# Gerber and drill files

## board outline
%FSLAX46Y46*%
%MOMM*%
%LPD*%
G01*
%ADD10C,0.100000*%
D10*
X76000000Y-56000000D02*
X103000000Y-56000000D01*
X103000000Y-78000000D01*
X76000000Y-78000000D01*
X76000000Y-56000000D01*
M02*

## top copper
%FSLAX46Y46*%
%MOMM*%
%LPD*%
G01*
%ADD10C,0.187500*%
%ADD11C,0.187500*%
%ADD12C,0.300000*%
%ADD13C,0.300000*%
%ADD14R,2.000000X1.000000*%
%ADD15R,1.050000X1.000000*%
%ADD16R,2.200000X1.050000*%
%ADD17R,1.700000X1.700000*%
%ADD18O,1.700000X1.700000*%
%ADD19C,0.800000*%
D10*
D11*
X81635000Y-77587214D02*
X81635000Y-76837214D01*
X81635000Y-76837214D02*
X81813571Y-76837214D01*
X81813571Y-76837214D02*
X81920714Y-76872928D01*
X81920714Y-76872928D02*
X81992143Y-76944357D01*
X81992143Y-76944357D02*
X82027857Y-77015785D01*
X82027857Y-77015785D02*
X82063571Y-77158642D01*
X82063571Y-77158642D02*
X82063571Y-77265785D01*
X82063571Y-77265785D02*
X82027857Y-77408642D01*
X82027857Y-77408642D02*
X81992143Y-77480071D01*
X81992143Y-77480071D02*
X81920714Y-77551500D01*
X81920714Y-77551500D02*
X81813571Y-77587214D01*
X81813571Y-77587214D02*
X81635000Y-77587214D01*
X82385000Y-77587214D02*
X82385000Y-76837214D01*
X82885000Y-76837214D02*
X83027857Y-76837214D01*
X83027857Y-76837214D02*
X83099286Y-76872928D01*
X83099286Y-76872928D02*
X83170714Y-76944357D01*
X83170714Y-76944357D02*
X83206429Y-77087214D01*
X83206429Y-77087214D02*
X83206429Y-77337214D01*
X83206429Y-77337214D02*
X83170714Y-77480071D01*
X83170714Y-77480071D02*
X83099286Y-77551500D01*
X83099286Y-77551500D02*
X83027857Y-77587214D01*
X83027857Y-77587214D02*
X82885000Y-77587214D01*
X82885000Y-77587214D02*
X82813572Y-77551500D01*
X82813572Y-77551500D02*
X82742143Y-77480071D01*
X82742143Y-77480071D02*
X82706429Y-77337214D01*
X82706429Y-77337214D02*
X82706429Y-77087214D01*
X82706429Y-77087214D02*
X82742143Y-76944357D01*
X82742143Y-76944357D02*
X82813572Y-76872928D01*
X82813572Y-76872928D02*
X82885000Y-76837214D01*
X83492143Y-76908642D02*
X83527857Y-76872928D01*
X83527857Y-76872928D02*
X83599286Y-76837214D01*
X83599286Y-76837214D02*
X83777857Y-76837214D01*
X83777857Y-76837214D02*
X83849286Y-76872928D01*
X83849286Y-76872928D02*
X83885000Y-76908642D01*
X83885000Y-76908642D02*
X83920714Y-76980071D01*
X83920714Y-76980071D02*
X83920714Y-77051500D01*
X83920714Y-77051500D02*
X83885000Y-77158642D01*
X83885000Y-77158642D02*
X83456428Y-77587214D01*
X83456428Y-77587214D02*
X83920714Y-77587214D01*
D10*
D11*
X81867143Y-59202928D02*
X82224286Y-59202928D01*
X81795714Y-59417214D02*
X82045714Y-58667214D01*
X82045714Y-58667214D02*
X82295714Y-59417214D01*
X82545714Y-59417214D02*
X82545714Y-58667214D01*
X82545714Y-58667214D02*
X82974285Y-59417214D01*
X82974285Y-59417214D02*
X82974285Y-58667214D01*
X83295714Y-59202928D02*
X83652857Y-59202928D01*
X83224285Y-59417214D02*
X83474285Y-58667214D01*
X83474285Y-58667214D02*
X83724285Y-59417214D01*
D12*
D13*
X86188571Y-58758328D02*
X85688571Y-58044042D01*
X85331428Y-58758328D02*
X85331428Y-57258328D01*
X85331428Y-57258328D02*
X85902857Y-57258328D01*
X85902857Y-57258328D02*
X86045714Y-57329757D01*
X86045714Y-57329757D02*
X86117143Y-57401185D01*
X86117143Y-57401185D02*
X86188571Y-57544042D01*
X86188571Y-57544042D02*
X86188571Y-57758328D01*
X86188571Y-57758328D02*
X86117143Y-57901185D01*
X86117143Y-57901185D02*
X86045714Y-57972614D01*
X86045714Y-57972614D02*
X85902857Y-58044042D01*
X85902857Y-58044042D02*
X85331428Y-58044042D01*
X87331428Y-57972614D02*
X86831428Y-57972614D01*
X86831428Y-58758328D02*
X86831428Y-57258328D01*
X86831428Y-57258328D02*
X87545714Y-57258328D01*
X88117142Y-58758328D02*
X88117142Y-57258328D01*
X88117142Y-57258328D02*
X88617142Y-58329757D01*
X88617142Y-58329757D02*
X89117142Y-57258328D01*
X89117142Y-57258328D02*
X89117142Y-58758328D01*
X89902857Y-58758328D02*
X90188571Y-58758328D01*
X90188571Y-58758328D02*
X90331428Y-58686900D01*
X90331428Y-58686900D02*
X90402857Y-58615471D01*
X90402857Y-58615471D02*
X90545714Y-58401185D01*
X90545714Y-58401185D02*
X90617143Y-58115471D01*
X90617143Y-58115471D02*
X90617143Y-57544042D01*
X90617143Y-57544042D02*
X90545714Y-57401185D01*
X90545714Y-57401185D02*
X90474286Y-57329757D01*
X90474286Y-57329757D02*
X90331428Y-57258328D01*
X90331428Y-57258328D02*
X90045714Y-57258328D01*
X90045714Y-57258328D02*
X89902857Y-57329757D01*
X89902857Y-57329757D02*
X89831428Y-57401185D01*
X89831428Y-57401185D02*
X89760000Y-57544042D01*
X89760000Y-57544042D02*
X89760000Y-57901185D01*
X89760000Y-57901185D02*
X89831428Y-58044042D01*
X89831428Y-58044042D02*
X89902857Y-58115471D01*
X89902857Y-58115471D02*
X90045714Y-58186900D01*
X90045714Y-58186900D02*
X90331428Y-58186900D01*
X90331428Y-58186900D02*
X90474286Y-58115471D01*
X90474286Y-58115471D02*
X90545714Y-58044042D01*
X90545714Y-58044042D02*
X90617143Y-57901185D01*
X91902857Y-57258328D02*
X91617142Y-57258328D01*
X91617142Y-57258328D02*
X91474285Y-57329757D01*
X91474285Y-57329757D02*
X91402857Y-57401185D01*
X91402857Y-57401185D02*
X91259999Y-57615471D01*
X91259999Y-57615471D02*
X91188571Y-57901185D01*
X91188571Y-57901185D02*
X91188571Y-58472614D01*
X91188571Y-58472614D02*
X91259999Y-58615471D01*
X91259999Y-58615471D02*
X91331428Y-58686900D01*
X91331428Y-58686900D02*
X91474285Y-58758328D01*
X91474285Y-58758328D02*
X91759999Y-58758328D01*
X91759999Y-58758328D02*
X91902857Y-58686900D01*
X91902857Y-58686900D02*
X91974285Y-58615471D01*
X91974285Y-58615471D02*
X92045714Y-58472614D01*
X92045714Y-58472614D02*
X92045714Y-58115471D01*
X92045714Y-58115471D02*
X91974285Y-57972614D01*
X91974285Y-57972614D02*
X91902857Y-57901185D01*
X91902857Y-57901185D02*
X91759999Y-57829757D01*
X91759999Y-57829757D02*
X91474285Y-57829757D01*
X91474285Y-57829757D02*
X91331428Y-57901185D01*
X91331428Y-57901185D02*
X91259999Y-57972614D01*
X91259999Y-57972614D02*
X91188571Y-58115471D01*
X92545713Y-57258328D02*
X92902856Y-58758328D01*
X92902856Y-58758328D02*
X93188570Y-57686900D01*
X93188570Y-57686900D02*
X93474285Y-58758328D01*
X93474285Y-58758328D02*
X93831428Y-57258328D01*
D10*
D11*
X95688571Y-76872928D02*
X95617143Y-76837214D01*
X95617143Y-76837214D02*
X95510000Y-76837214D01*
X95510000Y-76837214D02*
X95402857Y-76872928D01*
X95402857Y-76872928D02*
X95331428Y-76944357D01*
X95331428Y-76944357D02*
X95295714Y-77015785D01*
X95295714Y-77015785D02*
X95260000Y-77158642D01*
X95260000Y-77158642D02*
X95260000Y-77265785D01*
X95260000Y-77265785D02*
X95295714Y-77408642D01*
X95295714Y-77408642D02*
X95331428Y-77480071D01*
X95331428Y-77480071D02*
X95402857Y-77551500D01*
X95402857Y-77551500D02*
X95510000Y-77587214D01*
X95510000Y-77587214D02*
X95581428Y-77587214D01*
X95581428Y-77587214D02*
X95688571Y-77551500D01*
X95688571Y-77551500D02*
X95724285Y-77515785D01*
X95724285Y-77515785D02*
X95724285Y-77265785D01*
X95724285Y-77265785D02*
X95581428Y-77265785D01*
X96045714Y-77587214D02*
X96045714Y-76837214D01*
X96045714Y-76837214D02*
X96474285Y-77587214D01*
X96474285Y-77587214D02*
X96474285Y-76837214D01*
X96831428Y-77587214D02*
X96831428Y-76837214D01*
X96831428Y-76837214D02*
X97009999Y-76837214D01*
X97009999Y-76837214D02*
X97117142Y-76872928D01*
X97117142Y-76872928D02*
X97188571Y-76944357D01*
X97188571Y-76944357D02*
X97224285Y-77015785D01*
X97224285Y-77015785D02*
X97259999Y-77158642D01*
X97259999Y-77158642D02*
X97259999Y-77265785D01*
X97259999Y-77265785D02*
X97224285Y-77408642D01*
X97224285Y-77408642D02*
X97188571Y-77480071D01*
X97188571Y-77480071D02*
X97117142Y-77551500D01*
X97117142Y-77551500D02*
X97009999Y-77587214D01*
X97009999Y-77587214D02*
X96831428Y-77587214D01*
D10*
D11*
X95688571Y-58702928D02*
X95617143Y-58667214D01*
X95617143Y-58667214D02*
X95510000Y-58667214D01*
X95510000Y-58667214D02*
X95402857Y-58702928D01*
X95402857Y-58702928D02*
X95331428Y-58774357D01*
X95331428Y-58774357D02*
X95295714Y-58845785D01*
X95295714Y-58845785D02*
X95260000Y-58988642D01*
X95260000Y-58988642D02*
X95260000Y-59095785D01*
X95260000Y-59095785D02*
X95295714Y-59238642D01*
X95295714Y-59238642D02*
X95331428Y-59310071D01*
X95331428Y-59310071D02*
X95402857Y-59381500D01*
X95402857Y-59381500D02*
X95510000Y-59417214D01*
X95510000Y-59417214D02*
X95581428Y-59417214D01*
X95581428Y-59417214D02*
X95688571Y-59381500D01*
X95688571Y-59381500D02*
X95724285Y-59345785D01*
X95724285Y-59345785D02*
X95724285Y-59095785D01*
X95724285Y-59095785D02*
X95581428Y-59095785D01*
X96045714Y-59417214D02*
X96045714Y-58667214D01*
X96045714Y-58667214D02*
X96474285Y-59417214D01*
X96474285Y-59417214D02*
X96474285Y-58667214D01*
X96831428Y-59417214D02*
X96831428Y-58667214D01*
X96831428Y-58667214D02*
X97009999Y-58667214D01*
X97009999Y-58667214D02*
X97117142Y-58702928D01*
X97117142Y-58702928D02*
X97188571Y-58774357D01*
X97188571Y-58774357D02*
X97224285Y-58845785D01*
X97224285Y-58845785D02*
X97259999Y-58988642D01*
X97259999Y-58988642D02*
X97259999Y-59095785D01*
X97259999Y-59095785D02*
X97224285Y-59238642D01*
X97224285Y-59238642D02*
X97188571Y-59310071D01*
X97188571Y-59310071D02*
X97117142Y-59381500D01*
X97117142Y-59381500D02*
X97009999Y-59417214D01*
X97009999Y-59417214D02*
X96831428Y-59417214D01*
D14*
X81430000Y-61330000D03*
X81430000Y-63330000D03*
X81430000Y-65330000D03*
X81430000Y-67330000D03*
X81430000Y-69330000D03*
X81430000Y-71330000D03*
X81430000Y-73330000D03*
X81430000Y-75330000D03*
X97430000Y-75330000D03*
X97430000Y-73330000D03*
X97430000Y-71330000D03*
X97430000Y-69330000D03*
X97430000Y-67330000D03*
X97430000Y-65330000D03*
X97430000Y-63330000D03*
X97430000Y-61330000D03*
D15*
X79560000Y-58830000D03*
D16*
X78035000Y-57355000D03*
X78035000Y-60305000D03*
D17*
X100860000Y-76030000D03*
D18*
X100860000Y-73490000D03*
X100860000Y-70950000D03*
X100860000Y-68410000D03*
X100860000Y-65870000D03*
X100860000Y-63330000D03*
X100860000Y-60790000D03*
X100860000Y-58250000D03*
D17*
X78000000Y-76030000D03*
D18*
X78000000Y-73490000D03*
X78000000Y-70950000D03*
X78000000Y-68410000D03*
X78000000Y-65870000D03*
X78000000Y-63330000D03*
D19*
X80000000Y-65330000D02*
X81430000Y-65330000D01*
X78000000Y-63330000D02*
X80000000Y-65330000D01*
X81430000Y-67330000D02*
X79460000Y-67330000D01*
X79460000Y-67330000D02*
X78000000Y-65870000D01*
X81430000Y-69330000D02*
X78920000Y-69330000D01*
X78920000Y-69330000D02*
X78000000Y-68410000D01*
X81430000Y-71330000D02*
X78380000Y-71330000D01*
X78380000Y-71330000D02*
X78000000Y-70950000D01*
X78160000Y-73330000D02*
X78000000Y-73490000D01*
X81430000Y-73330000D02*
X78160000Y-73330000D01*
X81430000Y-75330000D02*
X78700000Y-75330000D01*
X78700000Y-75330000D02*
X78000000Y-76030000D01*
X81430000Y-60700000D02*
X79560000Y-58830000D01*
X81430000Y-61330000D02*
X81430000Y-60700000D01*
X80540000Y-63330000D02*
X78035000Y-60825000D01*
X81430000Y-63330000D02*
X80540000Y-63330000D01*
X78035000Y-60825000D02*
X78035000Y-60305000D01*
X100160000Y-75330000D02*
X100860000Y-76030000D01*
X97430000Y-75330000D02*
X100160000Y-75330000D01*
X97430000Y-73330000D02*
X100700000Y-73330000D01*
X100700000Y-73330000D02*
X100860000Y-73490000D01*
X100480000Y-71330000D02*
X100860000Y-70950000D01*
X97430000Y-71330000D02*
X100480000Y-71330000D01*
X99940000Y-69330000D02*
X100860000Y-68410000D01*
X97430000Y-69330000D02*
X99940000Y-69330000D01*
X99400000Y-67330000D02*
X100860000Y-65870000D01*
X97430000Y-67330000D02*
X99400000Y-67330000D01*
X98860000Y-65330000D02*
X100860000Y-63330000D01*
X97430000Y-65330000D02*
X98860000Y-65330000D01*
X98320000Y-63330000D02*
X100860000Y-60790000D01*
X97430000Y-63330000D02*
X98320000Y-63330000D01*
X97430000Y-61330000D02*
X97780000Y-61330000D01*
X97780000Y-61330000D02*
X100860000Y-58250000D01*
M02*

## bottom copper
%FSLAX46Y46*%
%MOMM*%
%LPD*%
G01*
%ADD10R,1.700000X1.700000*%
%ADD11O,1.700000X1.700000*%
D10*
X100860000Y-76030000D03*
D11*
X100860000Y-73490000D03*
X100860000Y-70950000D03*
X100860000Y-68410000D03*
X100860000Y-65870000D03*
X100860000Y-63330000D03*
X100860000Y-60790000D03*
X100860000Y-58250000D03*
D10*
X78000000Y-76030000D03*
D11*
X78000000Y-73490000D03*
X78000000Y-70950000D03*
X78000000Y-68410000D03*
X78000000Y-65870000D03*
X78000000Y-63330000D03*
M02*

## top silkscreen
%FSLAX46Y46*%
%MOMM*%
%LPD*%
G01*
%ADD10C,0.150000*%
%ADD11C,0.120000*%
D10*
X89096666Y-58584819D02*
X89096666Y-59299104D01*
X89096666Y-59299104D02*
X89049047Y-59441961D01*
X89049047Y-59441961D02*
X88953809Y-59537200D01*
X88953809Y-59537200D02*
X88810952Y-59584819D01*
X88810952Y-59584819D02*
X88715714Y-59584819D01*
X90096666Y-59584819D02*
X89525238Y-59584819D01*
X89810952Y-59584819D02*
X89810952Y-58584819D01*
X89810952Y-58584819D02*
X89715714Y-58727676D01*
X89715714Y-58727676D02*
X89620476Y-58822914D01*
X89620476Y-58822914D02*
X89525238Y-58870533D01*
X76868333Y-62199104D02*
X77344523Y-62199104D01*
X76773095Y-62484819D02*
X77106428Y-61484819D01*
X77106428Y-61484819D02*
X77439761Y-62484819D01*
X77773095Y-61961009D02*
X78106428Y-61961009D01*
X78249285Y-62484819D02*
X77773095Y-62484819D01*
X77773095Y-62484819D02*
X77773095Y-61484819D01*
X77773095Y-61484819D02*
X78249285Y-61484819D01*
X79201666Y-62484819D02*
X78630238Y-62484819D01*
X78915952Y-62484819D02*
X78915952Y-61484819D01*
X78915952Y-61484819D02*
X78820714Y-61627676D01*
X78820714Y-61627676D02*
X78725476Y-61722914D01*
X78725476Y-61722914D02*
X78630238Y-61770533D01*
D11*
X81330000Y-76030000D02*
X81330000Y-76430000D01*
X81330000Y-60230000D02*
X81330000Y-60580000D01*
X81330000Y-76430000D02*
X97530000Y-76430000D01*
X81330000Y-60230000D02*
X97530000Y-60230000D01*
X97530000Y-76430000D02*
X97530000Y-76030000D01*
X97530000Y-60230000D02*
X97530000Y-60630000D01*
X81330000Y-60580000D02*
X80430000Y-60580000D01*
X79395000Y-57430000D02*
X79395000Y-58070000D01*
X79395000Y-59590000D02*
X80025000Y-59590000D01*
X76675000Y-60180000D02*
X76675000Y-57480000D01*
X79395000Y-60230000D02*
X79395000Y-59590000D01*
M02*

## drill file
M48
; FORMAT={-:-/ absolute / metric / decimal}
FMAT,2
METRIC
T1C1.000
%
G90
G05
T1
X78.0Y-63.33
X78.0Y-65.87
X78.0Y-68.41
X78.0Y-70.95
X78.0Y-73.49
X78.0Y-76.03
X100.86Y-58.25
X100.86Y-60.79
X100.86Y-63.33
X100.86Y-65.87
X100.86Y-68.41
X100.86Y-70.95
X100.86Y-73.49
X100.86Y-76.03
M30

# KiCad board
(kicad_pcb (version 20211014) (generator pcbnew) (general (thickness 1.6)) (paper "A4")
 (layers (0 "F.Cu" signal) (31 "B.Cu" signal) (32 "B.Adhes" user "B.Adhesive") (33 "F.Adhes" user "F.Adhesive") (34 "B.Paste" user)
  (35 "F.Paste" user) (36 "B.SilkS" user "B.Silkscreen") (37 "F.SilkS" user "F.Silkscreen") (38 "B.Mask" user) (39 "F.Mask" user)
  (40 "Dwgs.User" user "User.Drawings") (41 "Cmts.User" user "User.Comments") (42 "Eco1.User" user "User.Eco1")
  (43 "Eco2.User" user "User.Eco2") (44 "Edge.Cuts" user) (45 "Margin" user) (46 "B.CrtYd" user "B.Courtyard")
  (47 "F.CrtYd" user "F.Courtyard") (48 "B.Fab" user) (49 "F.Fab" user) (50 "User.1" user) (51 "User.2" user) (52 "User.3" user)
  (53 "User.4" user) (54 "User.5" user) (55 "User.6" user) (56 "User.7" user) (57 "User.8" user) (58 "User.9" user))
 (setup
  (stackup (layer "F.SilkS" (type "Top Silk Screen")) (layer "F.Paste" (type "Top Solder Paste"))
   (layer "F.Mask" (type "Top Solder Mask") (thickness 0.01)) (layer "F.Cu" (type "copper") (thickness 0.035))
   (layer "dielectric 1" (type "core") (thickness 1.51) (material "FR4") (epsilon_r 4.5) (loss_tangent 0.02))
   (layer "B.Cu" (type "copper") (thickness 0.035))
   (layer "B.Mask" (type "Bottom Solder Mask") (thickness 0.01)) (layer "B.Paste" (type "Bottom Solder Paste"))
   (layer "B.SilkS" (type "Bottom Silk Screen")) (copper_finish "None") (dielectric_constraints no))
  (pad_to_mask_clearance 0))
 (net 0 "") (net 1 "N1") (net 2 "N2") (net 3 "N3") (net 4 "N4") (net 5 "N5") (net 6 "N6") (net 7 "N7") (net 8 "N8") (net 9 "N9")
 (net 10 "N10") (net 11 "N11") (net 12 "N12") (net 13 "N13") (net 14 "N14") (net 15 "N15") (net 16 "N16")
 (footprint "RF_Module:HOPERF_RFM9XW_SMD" (layer "F.Cu") (at 89.43 68.33)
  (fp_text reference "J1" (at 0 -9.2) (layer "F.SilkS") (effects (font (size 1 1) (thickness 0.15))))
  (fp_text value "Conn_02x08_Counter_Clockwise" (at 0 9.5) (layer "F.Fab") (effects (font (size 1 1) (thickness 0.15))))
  (fp_line (start -8.1 7.7) (end -8.1 8.1) (layer "F.SilkS") (width 0.12))
  (fp_line (start -8.1 -8.1) (end -8.1 -7.75) (layer "F.SilkS") (width 0.12))
  (fp_line (start -8.1 8.1) (end 8.1 8.1) (layer "F.SilkS") (width 0.12))
  (fp_line (start -8.1 -8.1) (end 8.1 -8.1) (layer "F.SilkS") (width 0.12))
  (fp_line (start 8.1 8.1) (end 8.1 7.7) (layer "F.SilkS") (width 0.12))
  (fp_line (start 8.1 -8.1) (end 8.1 -7.7) (layer "F.SilkS") (width 0.12))
  (fp_line (start -8.1 -7.75) (end -9 -7.75) (layer "F.SilkS") (width 0.12))
  (pad "1" smd rect (at -8 -7) (size 2 1) (layers "F.Cu" "F.Paste" "F.Mask") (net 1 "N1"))
  (pad "2" smd rect (at -8 -5) (size 2 1) (layers "F.Cu" "F.Paste" "F.Mask") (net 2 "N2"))
  (pad "3" smd rect (at -8 -3) (size 2 1) (layers "F.Cu" "F.Paste" "F.Mask") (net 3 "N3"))
  (pad "4" smd rect (at -8 -1) (size 2 1) (layers "F.Cu" "F.Paste" "F.Mask") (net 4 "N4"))
  (pad "5" smd rect (at -8 1) (size 2 1) (layers "F.Cu" "F.Paste" "F.Mask") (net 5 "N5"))
  (pad "6" smd rect (at -8 3) (size 2 1) (layers "F.Cu" "F.Paste" "F.Mask") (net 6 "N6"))
  (pad "7" smd rect (at -8 5) (size 2 1) (layers "F.Cu" "F.Paste" "F.Mask") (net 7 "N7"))
  (pad "8" smd rect (at -8 7) (size 2 1) (layers "F.Cu" "F.Paste" "F.Mask") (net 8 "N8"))
  (pad "9" smd rect (at 8 7) (size 2 1) (layers "F.Cu" "F.Paste" "F.Mask") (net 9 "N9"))
  (pad "10" smd rect (at 8 5) (size 2 1) (layers "F.Cu" "F.Paste" "F.Mask") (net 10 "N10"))
  (pad "11" smd rect (at 8 3) (size 2 1) (layers "F.Cu" "F.Paste" "F.Mask") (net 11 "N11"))
  (pad "12" smd rect (at 8 1) (size 2 1) (layers "F.Cu" "F.Paste" "F.Mask") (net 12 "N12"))
  (pad "13" smd rect (at 8 -1) (size 2 1) (layers "F.Cu" "F.Paste" "F.Mask") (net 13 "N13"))
  (pad "14" smd rect (at 8 -3) (size 2 1) (layers "F.Cu" "F.Paste" "F.Mask") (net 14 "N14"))
  (pad "15" smd rect (at 8 -5) (size 2 1) (layers "F.Cu" "F.Paste" "F.Mask") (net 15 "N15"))
  (pad "16" smd rect (at 8 -7) (size 2 1) (layers "F.Cu" "F.Paste" "F.Mask") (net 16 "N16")))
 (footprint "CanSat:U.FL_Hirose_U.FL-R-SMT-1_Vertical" (layer "F.Cu") (at 78.51 58.83 180)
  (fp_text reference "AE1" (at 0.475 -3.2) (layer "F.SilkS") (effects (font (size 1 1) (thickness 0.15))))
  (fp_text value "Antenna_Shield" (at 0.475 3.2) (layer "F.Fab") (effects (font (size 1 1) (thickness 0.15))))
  (fp_line (start -0.885 1.4) (end -0.885 0.76) (layer "F.SilkS") (width 0.12))
  (fp_line (start -0.885 -0.76) (end -1.515 -0.76) (layer "F.SilkS") (width 0.12))
  (fp_line (start 1.835 -1.35) (end 1.835 1.35) (layer "F.SilkS") (width 0.12))
  (fp_line (start -0.885 -1.4) (end -0.885 -0.76) (layer "F.SilkS") (width 0.12))
  (pad "1" smd rect (at -1.05 0 180) (size 1.05 1) (layers "F.Cu" "F.Paste" "F.Mask") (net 1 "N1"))
  (pad "2" smd rect (at 0.475 1.475 180) (size 2.2 1.05) (layers "F.Cu" "F.Paste" "F.Mask") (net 2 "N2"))
  (pad "2" smd rect (at 0.475 -1.475 180) (size 2.2 1.05) (layers "F.Cu" "F.Paste" "F.Mask") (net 2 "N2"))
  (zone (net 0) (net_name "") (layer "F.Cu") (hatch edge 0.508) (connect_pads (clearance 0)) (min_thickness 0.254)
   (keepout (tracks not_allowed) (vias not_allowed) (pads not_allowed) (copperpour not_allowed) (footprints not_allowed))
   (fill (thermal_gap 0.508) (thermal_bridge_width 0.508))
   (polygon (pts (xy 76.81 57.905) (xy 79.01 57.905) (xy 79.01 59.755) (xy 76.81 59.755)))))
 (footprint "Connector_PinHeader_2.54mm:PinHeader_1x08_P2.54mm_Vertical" (layer "B.Cu") (at 100.86 76.03)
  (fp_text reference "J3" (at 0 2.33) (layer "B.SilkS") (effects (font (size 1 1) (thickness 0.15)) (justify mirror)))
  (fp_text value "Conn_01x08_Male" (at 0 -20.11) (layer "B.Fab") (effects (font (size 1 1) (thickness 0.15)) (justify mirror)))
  (pad "1" thru_hole rect (at 0 0) (size 1.7 1.7) (drill 1) (layers *.Cu *.Mask) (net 9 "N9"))
  (pad "2" thru_hole oval (at 0 -2.54) (size 1.7 1.7) (drill 1) (layers *.Cu *.Mask) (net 10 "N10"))
  (pad "3" thru_hole oval (at 0 -5.08) (size 1.7 1.7) (drill 1) (layers *.Cu *.Mask) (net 11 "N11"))
  (pad "4" thru_hole oval (at 0 -7.62) (size 1.7 1.7) (drill 1) (layers *.Cu *.Mask) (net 12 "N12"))
  (pad "5" thru_hole oval (at 0 -10.16) (size 1.7 1.7) (drill 1) (layers *.Cu *.Mask) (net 13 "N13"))
  (pad "6" thru_hole oval (at 0 -12.7) (size 1.7 1.7) (drill 1) (layers *.Cu *.Mask) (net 14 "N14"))
  (pad "7" thru_hole oval (at 0 -15.24) (size 1.7 1.7) (drill 1) (layers *.Cu *.Mask) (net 15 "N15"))
  (pad "8" thru_hole oval (at 0 -17.78) (size 1.7 1.7) (drill 1) (layers *.Cu *.Mask) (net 16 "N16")))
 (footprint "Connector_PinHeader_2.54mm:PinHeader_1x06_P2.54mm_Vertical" (layer "B.Cu") (at 78 76.03)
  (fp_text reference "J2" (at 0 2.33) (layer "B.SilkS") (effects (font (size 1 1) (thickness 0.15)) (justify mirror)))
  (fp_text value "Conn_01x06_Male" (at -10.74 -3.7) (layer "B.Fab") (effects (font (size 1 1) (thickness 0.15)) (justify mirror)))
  (pad "1" thru_hole rect (at 0 0) (size 1.7 1.7) (drill 1) (layers *.Cu *.Mask) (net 8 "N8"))
  (pad "2" thru_hole oval (at 0 -2.54) (size 1.7 1.7) (drill 1) (layers *.Cu *.Mask) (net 7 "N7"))
  (pad "3" thru_hole oval (at 0 -5.08) (size 1.7 1.7) (drill 1) (layers *.Cu *.Mask) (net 6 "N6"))
  (pad "4" thru_hole oval (at 0 -7.62) (size 1.7 1.7) (drill 1) (layers *.Cu *.Mask) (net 5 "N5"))
  (pad "5" thru_hole oval (at 0 -10.16) (size 1.7 1.7) (drill 1) (layers *.Cu *.Mask) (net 4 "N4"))
  (pad "6" thru_hole oval (at 0 -12.7) (size 1.7 1.7) (drill 1) (layers *.Cu *.Mask) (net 3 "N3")))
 (gr_rect (start 76 56) (end 103 78) (layer "Edge.Cuts") (width 0.1) (fill none))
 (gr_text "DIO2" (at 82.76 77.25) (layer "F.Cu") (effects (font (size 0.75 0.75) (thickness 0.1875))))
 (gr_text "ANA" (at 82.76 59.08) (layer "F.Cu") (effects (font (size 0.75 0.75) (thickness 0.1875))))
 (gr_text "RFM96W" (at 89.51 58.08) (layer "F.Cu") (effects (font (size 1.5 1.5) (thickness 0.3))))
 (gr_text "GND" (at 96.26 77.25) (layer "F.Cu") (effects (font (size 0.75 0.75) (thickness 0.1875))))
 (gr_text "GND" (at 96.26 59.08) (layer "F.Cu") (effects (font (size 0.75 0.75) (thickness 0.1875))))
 (segment (start 80 65.33) (end 81.43 65.33) (width 0.8) (layer "F.Cu") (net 3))
 (segment (start 78 63.33) (end 80 65.33) (width 0.8) (layer "F.Cu") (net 3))
 (segment (start 81.43 67.33) (end 79.46 67.33) (width 0.8) (layer "F.Cu") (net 4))
 (segment (start 79.46 67.33) (end 78 65.87) (width 0.8) (layer "F.Cu") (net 4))
 (segment (start 81.43 69.33) (end 78.92 69.33) (width 0.8) (layer "F.Cu") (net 5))
 (segment (start 78.92 69.33) (end 78 68.41) (width 0.8) (layer "F.Cu") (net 5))
 (segment (start 81.43 71.33) (end 78.38 71.33) (width 0.8) (layer "F.Cu") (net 6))
 (segment (start 78.38 71.33) (end 78 70.95) (width 0.8) (layer "F.Cu") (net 6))
 (segment (start 78.16 73.33) (end 78 73.49) (width 0.8) (layer "F.Cu") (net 7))
 (segment (start 81.43 73.33) (end 78.16 73.33) (width 0.8) (layer "F.Cu") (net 7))
 (segment (start 81.43 75.33) (end 78.7 75.33) (width 0.8) (layer "F.Cu") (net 8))
 (segment (start 78.7 75.33) (end 78 76.03) (width 0.8) (layer "F.Cu") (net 8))
 (segment (start 81.43 60.7) (end 79.56 58.83) (width 0.8) (layer "F.Cu") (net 1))
 (segment (start 81.43 61.33) (end 81.43 60.7) (width 0.8) (layer "F.Cu") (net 1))
 (segment (start 80.54 63.33) (end 78.035 60.825) (width 0.8) (layer "F.Cu") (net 2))
 (segment (start 81.43 63.33) (end 80.54 63.33) (width 0.8) (layer "F.Cu") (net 2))
 (segment (start 78.035 60.825) (end 78.035 60.305) (width 0.8) (layer "F.Cu") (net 2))
 (segment (start 100.16 75.33) (end 100.86 76.03) (width 0.8) (layer "F.Cu") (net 9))
 (segment (start 97.43 75.33) (end 100.16 75.33) (width 0.8) (layer "F.Cu") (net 9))
 (segment (start 97.43 73.33) (end 100.7 73.33) (width 0.8) (layer "F.Cu") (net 10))
 (segment (start 100.7 73.33) (end 100.86 73.49) (width 0.8) (layer "F.Cu") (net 10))
 (segment (start 100.48 71.33) (end 100.86 70.95) (width 0.8) (layer "F.Cu") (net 11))
 (segment (start 97.43 71.33) (end 100.48 71.33) (width 0.8) (layer "F.Cu") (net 11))
 (segment (start 99.94 69.33) (end 100.86 68.41) (width 0.8) (layer "F.Cu") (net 12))
 (segment (start 97.43 69.33) (end 99.94 69.33) (width 0.8) (layer "F.Cu") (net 12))
 (segment (start 99.4 67.33) (end 100.86 65.87) (width 0.8) (layer "F.Cu") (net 13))
 (segment (start 97.43 67.33) (end 99.4 67.33) (width 0.8) (layer "F.Cu") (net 13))
 (segment (start 98.86 65.33) (end 100.86 63.33) (width 0.8) (layer "F.Cu") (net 14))
 (segment (start 97.43 65.33) (end 98.86 65.33) (width 0.8) (layer "F.Cu") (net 14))
 (segment (start 98.32 63.33) (end 100.86 60.79) (width 0.8) (layer "F.Cu") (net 15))
 (segment (start 97.43 63.33) (end 98.32 63.33) (width 0.8) (layer "F.Cu") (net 15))
 (segment (start 97.43 61.33) (end 97.78 61.33) (width 0.8) (layer "F.Cu") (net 16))
 (segment (start 97.78 61.33) (end 100.86 58.25) (width 0.8) (layer "F.Cu") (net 16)))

